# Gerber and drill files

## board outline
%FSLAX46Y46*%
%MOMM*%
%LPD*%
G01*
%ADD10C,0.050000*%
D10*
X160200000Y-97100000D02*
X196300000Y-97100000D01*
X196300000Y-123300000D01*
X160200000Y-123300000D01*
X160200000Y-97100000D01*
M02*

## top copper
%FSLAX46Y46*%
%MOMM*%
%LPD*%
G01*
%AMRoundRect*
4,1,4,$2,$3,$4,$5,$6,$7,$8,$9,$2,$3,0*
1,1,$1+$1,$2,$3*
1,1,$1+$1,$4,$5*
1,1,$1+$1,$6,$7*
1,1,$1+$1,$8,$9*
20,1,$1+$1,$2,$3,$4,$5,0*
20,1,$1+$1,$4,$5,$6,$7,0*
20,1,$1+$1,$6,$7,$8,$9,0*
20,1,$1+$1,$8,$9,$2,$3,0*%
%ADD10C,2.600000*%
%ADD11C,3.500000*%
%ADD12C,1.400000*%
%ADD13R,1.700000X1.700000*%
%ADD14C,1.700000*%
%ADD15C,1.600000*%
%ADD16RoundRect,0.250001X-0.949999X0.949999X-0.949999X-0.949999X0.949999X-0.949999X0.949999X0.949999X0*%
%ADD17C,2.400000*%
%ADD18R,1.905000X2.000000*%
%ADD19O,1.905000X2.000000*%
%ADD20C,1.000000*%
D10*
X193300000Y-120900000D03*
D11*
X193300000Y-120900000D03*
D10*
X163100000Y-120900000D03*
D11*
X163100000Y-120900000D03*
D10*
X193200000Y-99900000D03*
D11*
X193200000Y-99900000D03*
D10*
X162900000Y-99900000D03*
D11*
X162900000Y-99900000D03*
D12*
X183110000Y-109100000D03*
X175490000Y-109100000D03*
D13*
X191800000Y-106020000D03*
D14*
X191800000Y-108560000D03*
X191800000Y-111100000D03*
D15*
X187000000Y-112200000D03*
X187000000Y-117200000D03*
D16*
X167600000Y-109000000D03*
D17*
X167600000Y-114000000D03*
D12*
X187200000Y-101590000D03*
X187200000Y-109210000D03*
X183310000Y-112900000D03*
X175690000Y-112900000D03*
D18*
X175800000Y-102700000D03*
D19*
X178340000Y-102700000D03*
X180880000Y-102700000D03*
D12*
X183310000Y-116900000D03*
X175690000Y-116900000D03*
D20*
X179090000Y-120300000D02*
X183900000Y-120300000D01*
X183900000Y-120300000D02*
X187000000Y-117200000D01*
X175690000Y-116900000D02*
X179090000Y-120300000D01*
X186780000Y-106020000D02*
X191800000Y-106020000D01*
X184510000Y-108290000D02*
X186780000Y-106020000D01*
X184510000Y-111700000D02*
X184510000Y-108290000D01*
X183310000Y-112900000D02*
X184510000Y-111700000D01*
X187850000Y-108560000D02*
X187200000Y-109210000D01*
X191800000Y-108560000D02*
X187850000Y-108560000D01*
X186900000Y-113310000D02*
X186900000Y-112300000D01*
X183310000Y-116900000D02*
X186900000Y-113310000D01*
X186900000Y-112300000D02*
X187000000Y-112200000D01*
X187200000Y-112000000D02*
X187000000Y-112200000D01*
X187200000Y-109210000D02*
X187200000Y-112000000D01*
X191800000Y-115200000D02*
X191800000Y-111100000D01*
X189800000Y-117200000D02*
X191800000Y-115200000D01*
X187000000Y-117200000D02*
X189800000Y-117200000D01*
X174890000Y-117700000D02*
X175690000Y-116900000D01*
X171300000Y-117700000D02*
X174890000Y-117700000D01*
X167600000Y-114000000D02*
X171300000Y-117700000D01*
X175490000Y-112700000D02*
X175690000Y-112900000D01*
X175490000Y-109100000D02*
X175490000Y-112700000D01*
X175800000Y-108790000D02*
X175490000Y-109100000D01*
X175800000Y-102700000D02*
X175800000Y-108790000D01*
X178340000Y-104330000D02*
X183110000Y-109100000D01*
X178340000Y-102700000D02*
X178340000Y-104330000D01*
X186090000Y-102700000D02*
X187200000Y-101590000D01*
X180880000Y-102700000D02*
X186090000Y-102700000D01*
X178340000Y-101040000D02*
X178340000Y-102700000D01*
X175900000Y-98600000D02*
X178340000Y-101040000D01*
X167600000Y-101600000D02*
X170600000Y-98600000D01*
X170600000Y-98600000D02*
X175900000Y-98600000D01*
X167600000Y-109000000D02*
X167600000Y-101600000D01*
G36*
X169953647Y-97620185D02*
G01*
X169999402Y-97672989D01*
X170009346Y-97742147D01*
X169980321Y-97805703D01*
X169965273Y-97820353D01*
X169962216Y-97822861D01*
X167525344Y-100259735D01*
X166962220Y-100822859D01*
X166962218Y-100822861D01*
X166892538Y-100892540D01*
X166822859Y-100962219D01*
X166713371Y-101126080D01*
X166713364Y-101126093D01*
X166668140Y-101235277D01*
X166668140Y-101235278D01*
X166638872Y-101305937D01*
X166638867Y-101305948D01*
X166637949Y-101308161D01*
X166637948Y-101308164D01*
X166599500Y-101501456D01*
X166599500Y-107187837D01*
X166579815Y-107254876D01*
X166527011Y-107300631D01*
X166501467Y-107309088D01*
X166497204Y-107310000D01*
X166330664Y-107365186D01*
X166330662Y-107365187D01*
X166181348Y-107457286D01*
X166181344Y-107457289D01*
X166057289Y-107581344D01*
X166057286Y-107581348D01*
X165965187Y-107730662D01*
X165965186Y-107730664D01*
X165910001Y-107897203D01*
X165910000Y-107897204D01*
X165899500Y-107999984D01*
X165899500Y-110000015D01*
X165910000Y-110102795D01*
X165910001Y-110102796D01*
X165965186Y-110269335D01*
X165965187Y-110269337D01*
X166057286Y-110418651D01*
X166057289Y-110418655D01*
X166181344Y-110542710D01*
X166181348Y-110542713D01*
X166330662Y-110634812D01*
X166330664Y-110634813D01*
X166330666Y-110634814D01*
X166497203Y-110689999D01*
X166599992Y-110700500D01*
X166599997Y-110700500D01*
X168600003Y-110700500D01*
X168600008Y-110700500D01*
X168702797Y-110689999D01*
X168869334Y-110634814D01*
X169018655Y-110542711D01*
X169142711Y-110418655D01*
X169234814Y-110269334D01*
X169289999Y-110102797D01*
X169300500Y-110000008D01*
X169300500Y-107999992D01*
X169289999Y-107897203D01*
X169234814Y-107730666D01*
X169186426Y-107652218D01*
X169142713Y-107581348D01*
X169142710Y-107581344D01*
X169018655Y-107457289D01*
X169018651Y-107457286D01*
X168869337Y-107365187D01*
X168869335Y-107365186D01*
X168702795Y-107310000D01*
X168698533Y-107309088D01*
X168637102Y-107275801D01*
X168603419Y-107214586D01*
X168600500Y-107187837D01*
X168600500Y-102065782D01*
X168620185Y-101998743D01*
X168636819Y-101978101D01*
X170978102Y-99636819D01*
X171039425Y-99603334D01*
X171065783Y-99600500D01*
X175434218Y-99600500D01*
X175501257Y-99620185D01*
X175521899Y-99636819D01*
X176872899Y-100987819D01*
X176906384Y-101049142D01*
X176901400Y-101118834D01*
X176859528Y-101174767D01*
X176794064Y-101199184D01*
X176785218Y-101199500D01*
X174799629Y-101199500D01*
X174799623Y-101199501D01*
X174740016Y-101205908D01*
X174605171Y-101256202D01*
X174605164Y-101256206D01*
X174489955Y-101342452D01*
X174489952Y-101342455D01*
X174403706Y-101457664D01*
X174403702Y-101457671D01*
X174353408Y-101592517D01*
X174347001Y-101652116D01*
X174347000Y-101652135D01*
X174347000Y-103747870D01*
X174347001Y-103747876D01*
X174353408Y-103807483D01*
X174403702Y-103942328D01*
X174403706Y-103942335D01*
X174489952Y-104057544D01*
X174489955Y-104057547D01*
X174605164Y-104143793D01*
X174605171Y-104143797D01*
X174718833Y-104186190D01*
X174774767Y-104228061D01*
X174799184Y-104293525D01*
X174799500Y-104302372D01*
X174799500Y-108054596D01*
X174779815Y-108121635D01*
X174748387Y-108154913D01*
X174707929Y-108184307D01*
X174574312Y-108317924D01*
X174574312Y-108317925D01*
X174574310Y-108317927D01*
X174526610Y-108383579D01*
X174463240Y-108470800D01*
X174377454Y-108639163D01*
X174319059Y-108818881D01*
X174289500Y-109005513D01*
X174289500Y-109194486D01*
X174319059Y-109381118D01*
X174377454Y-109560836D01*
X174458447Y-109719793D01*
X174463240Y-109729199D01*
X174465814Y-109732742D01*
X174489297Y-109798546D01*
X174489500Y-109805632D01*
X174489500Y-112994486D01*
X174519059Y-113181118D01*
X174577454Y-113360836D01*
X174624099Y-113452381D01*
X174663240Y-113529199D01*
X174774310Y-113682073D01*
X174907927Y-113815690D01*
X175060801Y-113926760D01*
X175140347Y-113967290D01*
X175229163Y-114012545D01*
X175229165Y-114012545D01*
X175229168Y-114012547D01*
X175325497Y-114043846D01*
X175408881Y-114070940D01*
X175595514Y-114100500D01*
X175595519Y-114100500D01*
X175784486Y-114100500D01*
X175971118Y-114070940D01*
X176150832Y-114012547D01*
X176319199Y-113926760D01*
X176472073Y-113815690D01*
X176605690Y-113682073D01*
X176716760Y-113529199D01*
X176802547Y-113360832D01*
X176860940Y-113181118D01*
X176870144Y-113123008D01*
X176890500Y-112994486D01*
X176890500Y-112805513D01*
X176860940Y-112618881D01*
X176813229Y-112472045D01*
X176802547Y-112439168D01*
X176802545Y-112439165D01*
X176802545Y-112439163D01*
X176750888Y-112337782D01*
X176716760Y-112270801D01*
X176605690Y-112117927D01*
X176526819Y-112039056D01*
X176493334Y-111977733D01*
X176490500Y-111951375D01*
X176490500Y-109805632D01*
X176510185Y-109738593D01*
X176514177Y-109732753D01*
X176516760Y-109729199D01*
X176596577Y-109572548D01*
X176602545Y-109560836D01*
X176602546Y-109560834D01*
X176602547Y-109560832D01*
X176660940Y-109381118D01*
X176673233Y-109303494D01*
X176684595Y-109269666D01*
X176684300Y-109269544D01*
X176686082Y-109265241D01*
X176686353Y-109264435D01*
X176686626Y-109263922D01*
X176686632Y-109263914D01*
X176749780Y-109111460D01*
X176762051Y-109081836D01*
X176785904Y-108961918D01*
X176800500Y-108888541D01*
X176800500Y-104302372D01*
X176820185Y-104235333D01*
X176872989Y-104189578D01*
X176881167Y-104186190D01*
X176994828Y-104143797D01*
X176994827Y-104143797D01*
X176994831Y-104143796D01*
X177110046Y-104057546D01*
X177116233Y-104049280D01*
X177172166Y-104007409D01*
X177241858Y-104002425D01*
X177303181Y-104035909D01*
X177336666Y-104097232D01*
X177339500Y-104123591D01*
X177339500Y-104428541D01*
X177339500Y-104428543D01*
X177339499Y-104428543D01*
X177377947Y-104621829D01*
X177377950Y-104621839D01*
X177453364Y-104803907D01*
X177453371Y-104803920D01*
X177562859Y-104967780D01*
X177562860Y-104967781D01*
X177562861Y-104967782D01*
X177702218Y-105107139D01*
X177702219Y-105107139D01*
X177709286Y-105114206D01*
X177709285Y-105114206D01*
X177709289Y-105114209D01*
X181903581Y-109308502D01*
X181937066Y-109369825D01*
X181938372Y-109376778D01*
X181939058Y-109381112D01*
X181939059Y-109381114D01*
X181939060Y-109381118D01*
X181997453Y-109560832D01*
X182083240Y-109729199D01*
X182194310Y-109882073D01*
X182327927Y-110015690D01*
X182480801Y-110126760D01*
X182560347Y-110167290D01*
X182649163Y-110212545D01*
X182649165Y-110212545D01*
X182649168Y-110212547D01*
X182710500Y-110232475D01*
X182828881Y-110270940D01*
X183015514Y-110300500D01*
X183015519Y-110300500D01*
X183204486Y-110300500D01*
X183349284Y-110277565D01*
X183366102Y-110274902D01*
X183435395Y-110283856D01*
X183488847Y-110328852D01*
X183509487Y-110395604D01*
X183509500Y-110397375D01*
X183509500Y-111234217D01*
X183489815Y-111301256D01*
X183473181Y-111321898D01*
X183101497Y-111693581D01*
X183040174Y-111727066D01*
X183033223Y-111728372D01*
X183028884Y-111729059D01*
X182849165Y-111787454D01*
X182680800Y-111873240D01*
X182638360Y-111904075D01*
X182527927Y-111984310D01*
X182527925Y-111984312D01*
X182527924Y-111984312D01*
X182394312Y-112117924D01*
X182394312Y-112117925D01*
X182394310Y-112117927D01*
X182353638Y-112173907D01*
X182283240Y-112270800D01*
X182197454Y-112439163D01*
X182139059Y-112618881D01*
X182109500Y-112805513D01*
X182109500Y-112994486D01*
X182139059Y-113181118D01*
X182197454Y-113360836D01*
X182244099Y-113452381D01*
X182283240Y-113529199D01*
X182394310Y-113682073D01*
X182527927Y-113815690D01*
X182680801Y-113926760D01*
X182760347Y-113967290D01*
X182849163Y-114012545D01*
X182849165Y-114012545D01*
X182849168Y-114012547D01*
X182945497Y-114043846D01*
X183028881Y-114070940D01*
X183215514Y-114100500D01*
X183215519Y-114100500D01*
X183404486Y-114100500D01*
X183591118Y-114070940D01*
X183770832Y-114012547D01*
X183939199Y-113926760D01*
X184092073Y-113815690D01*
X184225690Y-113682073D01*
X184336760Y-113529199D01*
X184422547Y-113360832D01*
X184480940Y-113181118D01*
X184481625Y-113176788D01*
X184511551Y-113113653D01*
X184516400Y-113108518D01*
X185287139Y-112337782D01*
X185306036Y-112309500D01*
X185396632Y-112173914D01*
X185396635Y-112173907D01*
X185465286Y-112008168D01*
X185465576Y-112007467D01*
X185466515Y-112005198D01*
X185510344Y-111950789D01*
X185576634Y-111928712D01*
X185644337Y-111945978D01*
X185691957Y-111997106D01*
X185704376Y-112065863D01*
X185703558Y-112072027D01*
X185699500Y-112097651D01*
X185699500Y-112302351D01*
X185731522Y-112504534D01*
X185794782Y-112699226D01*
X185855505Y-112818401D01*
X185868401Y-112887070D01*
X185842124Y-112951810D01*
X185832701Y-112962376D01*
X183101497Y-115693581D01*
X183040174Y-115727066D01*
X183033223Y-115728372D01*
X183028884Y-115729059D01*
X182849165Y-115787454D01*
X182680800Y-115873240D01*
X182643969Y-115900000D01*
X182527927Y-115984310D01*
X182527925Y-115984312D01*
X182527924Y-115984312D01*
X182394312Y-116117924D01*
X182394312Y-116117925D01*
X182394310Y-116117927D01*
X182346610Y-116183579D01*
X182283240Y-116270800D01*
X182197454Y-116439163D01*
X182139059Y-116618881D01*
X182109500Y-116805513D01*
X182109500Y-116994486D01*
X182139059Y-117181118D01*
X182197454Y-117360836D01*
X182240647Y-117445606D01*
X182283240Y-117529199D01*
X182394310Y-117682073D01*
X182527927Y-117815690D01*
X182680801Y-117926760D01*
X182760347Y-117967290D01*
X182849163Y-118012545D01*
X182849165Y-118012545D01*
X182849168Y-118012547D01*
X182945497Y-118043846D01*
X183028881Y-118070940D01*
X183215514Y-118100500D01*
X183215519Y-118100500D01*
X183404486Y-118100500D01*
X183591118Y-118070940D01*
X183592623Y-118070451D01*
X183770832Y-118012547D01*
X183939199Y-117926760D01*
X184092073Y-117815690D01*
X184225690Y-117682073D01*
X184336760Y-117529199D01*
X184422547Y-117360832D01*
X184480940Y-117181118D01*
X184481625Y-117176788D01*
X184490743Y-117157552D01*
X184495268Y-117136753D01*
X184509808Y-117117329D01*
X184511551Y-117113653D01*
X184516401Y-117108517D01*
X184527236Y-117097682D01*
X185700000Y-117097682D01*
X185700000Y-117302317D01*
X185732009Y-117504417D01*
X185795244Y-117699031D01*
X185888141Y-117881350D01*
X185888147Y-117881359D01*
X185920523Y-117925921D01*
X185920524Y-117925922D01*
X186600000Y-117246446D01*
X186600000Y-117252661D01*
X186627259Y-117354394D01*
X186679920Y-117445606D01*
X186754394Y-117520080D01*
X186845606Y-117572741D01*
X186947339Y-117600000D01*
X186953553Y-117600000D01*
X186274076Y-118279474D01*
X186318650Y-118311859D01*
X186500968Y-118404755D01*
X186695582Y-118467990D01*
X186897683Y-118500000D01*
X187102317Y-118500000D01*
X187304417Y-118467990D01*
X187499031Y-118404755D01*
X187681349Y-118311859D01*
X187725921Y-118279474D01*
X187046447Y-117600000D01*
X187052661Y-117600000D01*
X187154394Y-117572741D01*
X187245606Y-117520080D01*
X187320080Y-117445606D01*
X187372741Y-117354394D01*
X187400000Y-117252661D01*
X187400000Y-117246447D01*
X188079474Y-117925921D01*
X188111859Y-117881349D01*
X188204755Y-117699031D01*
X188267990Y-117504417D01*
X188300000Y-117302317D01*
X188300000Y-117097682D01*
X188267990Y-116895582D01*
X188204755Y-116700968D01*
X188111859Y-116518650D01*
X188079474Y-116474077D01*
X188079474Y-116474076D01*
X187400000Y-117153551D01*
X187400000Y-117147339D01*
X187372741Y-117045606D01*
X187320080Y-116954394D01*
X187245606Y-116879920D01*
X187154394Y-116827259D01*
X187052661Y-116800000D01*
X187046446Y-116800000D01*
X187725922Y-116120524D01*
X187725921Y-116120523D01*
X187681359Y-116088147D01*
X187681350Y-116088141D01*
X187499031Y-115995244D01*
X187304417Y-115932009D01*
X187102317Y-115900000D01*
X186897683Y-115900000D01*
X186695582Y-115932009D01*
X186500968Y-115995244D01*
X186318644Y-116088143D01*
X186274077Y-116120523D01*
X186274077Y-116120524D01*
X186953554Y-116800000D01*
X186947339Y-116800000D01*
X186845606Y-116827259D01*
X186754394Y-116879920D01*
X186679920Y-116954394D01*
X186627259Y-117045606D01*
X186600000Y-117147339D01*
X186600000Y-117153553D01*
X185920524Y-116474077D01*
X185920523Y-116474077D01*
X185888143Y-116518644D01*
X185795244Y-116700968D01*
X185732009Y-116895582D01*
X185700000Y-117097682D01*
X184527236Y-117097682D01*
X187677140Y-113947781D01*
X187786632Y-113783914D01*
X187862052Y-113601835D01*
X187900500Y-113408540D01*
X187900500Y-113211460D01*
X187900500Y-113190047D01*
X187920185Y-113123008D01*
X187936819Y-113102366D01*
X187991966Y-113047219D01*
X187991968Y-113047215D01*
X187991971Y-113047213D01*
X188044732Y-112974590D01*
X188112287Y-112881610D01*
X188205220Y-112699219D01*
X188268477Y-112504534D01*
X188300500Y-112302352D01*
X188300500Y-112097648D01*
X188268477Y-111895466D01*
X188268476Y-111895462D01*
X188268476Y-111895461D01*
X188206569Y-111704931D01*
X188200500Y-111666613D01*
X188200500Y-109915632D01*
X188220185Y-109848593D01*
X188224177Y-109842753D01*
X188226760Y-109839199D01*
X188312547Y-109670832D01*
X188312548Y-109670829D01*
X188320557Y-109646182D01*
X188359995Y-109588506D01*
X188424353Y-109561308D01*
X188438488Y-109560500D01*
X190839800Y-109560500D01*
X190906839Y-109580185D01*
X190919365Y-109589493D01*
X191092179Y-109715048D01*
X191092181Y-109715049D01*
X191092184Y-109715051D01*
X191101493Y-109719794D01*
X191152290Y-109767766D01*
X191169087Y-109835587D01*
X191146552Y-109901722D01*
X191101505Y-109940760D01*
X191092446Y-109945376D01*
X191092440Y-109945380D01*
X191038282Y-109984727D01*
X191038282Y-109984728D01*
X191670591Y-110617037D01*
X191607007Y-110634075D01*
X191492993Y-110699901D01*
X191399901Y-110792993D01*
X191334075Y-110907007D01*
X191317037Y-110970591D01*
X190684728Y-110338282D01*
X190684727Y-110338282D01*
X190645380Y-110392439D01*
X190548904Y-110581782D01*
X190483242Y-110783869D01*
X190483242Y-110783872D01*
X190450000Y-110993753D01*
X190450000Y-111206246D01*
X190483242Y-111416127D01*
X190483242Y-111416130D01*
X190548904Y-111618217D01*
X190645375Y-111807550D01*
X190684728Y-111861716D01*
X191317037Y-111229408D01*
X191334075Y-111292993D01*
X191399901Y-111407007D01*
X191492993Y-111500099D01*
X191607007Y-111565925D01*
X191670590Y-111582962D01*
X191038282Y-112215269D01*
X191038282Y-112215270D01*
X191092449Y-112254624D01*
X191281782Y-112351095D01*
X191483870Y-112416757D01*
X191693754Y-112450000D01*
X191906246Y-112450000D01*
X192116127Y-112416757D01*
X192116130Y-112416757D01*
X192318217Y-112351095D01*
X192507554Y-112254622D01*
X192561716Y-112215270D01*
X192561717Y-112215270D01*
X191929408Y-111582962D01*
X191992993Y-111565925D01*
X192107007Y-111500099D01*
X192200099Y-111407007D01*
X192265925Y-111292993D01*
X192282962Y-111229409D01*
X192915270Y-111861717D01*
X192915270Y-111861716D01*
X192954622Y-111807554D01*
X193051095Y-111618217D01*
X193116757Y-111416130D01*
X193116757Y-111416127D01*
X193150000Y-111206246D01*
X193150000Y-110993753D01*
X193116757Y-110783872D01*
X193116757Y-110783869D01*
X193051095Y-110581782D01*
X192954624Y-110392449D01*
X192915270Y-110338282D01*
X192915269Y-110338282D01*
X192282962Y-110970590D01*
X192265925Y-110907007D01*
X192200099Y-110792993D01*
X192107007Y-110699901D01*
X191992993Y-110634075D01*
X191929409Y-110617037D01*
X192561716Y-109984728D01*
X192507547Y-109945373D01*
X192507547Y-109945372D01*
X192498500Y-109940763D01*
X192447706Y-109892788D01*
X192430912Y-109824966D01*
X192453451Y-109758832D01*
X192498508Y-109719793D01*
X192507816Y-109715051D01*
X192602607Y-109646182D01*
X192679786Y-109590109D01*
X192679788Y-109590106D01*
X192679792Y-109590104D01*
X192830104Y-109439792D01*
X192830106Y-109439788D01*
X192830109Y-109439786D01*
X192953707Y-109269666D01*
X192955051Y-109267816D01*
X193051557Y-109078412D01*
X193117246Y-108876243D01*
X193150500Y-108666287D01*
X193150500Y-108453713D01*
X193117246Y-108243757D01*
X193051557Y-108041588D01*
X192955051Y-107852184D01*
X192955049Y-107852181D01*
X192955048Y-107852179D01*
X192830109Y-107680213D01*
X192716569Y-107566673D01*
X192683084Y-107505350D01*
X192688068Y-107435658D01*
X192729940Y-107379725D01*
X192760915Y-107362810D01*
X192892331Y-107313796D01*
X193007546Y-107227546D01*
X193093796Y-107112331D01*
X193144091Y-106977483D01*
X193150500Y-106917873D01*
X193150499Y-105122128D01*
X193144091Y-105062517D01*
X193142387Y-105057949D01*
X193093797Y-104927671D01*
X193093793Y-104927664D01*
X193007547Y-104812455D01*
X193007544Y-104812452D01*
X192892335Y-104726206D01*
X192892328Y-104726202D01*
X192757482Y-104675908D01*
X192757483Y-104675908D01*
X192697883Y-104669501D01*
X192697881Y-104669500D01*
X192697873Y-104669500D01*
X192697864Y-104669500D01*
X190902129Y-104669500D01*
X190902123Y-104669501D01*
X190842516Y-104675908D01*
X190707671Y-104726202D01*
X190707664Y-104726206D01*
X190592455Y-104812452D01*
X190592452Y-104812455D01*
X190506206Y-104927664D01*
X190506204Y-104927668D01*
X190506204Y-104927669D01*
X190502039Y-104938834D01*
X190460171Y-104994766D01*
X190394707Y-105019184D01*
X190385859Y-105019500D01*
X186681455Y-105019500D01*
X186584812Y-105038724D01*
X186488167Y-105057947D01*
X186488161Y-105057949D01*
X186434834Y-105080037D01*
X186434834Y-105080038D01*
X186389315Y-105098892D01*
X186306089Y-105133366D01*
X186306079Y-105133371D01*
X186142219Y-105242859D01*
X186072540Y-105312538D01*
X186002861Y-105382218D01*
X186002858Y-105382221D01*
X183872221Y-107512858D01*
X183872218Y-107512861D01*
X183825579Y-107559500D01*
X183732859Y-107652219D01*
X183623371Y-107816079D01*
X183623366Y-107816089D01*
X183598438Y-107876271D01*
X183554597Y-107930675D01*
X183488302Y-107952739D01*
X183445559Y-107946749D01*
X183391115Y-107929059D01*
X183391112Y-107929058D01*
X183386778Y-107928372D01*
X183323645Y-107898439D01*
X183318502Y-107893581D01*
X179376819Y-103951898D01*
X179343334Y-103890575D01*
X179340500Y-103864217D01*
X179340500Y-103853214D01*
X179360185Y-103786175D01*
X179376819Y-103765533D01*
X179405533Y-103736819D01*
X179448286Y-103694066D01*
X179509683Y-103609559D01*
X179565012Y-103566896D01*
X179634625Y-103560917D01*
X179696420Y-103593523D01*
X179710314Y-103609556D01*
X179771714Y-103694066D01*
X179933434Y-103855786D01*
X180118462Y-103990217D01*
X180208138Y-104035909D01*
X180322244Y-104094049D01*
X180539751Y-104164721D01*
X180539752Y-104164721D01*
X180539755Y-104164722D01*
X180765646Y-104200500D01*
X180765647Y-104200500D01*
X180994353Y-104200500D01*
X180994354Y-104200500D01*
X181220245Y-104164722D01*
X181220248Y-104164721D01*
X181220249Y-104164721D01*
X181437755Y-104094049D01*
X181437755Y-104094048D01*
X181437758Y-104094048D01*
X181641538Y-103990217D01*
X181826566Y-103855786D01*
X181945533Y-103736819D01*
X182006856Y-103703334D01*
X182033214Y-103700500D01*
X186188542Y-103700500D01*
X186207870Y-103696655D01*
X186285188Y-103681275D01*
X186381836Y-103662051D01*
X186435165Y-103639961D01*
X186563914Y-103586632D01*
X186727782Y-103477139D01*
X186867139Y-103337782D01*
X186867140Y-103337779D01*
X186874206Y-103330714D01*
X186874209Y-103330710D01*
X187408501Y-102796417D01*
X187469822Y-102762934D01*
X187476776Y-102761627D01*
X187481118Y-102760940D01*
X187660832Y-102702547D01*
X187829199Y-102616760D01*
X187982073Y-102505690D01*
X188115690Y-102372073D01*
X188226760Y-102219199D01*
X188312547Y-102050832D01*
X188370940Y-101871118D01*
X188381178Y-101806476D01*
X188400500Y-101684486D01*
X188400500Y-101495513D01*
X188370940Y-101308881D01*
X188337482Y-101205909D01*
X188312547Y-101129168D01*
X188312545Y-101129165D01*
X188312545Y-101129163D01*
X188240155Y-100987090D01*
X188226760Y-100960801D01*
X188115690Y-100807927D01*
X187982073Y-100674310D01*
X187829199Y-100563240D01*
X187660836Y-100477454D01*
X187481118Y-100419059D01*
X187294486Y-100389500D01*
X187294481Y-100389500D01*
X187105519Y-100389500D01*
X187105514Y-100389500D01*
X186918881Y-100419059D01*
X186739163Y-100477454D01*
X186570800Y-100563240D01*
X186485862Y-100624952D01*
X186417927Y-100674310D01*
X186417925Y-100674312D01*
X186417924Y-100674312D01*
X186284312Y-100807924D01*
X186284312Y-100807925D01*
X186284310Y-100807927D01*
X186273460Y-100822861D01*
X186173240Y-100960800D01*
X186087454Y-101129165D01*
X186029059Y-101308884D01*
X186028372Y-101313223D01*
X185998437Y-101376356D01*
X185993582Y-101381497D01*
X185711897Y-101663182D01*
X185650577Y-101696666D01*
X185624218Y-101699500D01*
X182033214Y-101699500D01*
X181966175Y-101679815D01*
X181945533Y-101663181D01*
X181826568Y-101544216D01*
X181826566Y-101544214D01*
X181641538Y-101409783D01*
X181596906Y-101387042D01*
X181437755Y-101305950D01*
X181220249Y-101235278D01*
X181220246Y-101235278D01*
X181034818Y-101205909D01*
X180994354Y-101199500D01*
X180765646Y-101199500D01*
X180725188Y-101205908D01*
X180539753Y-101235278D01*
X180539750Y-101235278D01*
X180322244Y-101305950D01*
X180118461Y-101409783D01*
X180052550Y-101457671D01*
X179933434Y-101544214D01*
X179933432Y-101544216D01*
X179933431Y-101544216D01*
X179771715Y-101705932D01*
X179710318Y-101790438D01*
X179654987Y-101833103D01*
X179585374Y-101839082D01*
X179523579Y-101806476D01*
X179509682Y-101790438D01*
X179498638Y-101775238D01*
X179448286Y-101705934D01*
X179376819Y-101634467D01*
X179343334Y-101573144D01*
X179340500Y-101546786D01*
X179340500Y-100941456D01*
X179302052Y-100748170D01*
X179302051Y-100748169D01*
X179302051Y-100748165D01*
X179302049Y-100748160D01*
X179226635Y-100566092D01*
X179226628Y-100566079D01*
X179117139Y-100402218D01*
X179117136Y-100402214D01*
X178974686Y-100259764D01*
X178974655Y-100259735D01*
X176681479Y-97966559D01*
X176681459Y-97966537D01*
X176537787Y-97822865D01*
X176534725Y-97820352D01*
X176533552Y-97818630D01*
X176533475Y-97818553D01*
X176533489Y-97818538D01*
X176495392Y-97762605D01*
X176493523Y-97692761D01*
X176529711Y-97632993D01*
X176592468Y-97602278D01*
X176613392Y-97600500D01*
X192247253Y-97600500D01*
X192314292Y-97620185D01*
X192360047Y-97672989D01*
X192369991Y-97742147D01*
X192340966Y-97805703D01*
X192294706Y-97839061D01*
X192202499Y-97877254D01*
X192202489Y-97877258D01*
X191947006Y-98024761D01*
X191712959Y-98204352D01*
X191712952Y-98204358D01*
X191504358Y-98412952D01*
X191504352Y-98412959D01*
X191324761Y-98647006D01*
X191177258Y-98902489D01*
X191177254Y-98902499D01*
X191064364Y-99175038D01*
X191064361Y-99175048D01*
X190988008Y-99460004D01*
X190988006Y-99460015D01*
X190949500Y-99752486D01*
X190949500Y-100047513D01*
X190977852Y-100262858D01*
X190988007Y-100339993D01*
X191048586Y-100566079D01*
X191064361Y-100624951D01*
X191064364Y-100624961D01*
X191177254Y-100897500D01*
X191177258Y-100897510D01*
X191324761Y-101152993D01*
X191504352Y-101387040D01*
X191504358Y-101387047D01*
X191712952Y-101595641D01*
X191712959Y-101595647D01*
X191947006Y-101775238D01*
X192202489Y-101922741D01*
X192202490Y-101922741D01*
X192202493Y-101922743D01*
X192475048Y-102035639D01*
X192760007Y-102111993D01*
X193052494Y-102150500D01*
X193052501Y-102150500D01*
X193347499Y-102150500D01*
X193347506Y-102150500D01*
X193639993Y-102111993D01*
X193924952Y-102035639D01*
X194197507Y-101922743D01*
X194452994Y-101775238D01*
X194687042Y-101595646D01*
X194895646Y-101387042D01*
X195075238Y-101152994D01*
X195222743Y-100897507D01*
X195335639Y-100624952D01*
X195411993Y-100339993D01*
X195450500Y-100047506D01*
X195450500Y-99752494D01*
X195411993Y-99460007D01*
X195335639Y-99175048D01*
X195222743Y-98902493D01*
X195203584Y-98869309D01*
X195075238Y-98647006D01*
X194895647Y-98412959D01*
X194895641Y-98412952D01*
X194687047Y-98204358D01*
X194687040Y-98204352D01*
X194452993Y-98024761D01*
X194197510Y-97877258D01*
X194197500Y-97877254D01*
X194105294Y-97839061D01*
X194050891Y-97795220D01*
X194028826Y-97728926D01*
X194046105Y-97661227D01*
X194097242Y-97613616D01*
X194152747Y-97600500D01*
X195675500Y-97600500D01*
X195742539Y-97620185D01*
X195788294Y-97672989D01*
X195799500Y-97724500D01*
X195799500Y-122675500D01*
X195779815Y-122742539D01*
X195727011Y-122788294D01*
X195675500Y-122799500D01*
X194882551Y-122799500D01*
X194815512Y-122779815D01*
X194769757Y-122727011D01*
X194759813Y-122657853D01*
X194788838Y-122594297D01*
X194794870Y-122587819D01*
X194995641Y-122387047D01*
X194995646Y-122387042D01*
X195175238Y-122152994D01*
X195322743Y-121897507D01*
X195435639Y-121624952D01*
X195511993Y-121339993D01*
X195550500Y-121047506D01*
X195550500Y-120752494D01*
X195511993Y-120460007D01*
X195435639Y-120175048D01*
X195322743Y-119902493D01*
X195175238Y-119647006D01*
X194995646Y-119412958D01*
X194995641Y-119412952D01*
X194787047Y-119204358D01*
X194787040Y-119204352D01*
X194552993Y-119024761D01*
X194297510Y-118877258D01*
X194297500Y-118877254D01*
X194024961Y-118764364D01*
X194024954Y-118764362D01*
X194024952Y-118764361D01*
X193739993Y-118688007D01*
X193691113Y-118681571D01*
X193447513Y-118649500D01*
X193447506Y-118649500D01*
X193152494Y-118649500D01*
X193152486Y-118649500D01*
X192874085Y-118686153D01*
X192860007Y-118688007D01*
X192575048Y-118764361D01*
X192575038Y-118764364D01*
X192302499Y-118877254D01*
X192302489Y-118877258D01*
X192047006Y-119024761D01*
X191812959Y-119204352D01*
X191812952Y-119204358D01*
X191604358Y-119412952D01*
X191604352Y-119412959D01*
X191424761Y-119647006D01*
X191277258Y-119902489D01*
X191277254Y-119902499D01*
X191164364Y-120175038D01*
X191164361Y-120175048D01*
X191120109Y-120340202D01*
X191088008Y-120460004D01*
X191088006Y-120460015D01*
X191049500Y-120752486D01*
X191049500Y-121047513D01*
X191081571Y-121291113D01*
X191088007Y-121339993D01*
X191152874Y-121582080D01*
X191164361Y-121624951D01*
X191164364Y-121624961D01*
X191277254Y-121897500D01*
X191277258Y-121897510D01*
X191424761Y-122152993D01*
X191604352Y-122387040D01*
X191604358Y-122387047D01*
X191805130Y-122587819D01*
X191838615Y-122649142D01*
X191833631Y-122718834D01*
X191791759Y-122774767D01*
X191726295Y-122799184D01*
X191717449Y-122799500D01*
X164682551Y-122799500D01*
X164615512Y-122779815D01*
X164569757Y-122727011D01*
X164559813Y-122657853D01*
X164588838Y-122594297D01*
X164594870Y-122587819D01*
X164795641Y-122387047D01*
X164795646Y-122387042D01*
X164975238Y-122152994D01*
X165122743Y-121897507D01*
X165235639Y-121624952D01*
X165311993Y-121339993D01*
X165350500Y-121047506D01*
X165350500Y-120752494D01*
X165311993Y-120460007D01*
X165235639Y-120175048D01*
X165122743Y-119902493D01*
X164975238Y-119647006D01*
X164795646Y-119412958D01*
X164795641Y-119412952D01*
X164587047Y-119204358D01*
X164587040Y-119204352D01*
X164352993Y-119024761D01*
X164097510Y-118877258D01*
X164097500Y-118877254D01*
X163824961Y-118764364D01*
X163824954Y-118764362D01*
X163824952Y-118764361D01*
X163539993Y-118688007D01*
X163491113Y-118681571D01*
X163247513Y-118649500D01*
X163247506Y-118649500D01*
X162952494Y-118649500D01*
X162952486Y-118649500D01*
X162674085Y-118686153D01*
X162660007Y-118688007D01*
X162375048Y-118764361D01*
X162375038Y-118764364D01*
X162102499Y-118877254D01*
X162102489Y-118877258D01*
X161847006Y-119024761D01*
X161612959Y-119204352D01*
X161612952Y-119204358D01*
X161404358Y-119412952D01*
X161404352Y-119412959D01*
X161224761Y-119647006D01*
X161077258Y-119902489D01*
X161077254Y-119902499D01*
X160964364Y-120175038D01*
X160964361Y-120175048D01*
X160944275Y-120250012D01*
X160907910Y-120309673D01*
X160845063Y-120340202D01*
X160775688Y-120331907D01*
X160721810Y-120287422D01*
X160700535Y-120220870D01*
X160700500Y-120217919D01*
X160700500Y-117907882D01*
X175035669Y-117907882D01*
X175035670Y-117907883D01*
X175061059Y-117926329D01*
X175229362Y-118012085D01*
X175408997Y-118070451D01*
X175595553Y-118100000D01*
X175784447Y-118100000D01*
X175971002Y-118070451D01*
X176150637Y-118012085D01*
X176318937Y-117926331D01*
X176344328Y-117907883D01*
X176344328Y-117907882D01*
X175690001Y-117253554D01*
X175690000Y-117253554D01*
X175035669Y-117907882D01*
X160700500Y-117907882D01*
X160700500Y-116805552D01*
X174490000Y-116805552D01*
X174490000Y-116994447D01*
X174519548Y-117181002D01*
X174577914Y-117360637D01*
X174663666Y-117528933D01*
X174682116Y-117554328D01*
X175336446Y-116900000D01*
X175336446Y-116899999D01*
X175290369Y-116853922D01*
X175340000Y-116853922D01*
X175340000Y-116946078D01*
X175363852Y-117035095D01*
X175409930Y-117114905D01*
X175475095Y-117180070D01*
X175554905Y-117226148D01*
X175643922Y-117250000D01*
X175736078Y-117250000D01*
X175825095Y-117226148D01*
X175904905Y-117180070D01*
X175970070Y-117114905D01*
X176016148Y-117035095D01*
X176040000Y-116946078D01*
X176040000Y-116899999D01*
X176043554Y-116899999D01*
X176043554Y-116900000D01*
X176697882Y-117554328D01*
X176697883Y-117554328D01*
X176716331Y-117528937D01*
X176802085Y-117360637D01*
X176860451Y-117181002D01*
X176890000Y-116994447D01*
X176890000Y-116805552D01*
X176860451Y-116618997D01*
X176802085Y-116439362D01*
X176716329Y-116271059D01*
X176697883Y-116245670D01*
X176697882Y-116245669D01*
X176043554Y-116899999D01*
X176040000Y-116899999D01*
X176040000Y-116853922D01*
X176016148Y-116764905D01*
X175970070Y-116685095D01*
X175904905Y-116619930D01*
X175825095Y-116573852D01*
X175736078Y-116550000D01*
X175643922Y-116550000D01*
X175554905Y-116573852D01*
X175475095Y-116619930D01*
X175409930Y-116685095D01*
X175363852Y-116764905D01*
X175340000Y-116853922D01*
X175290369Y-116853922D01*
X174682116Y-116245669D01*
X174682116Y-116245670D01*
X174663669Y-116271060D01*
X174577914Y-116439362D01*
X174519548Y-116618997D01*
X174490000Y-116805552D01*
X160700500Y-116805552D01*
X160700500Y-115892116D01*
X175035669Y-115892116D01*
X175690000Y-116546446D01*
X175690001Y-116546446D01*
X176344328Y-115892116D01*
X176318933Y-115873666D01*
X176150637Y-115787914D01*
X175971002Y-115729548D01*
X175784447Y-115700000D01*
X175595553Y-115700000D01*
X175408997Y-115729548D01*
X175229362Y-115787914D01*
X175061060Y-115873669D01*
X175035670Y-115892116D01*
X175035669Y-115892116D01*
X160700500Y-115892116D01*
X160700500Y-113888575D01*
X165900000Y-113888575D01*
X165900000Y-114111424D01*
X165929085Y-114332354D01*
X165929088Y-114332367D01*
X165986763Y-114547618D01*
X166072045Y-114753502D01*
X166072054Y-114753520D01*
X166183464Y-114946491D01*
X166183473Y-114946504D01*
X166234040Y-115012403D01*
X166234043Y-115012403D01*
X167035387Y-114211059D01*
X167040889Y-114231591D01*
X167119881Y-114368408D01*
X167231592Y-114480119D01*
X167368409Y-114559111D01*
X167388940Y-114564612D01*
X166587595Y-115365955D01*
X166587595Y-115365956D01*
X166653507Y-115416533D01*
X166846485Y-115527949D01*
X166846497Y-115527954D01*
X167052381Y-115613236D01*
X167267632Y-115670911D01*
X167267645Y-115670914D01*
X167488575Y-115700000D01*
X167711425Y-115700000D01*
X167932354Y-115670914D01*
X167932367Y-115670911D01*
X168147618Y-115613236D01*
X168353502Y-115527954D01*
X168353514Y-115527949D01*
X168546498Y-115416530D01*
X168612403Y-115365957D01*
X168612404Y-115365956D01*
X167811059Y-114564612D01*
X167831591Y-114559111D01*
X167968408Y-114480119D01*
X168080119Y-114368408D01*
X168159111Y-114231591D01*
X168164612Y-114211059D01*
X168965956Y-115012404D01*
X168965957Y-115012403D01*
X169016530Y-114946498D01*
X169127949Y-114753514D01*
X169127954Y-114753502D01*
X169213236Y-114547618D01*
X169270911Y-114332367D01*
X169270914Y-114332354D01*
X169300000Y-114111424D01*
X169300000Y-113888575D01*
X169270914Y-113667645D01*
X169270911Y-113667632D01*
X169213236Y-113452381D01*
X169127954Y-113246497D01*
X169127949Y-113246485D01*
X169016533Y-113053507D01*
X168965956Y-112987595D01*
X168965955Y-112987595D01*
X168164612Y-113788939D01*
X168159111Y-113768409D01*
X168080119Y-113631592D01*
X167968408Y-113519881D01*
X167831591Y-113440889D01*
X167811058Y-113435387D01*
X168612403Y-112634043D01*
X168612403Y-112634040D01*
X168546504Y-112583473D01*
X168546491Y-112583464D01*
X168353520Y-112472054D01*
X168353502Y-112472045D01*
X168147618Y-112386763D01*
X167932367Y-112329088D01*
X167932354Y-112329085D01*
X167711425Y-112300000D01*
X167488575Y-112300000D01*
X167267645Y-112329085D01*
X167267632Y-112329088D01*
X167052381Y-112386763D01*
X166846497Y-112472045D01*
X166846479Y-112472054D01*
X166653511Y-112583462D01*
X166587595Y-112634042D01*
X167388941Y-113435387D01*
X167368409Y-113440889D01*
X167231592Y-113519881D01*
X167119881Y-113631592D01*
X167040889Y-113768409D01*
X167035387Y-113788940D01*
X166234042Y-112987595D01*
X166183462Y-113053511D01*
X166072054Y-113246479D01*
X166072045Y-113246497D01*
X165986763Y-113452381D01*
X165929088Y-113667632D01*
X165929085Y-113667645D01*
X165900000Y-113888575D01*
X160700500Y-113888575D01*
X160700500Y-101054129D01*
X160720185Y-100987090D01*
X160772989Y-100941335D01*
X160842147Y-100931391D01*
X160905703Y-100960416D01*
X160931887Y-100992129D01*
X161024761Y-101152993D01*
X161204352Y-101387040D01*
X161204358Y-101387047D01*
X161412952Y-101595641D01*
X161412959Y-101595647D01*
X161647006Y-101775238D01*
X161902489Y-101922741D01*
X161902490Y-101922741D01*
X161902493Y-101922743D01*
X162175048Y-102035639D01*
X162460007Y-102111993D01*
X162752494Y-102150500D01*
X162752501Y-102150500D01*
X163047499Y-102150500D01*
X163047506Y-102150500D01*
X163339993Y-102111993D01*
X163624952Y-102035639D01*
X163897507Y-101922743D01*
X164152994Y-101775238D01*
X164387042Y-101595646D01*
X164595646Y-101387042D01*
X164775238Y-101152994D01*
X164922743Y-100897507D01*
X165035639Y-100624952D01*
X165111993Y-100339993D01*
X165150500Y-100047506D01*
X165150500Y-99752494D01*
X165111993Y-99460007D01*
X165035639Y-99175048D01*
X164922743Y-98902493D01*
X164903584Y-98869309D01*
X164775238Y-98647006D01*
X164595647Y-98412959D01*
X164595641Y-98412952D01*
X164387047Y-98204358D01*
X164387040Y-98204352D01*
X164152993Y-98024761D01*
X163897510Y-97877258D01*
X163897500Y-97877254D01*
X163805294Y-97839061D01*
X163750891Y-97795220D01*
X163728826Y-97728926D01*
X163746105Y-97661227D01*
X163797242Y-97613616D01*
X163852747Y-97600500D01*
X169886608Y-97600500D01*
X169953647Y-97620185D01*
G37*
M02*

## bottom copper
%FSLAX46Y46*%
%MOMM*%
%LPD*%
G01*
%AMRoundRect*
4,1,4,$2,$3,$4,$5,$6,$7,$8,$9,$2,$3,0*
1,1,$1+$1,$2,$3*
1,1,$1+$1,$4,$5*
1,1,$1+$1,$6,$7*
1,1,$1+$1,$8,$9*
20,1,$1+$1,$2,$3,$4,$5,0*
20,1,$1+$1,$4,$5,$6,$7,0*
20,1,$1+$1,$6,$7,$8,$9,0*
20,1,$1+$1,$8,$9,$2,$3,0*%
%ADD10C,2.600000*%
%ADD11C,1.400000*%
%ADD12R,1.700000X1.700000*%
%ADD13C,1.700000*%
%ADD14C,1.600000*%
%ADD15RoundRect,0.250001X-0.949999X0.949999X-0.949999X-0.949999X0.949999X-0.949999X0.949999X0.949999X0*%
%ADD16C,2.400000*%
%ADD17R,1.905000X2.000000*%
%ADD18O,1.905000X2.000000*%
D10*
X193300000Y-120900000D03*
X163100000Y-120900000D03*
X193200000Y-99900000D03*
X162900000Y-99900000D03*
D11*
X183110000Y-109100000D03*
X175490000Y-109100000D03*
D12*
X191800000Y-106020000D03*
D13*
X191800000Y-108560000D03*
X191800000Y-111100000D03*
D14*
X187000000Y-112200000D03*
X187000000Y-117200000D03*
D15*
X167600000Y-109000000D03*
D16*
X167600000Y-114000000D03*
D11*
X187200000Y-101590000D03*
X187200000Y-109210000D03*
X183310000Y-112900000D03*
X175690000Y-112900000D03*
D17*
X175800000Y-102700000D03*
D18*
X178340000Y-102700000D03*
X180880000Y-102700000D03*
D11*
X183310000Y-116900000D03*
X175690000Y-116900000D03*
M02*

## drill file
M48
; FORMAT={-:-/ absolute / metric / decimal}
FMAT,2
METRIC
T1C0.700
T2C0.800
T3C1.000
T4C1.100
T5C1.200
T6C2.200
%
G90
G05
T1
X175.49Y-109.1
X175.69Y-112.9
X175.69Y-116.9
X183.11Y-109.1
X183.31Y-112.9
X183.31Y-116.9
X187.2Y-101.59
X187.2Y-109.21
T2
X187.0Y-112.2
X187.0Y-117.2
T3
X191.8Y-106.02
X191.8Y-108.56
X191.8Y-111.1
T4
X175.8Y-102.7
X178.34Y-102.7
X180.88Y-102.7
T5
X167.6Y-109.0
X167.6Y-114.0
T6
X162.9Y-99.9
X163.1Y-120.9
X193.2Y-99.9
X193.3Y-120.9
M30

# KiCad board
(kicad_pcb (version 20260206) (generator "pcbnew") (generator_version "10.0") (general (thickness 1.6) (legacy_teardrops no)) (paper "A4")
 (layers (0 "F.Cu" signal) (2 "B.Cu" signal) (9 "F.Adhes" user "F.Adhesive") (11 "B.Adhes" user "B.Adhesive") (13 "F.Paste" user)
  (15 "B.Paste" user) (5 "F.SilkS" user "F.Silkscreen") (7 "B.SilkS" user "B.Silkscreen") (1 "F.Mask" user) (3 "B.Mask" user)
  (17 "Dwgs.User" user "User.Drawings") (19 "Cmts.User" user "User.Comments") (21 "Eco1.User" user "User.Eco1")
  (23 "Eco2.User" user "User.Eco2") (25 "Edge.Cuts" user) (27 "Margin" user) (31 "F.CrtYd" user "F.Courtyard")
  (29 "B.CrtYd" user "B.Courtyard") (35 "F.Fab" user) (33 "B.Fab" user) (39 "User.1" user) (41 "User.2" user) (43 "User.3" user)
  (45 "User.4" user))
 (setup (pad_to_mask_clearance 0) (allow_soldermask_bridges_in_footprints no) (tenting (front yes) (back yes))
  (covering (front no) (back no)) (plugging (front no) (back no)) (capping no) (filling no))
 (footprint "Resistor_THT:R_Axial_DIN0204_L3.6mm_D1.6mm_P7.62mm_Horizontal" (layer "F.Cu") (at 183.11 109.1 180)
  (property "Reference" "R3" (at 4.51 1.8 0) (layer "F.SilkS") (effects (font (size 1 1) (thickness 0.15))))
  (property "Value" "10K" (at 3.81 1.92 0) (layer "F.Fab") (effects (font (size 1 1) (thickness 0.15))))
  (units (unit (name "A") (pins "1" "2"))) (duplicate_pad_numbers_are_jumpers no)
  (pad "1" thru_hole circle (at 0 0 180) (size 1.4 1.4) (drill 0.7) (layers "*.Cu" "*.Mask") (remove_unused_layers no)
   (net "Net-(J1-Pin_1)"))
  (pad "2" thru_hole circle (at 7.62 0 180) (size 1.4 1.4) (drill 0.7) (layers "*.Cu" "*.Mask") (remove_unused_layers no) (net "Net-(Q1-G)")))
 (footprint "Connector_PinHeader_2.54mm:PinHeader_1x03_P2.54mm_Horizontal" (layer "F.Cu") (at 191.8 106.02)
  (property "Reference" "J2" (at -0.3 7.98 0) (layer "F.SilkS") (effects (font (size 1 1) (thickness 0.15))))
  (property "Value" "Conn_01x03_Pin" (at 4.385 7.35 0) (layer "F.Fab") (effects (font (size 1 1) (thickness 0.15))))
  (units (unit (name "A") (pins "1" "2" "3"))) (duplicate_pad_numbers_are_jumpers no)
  (pad "1" thru_hole rect (at 0 0) (size 1.7 1.7) (drill 1) (layers "*.Cu" "*.Mask") (remove_unused_layers no) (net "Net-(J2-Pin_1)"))
  (pad "2" thru_hole circle (at 0 2.54) (size 1.7 1.7) (drill 1) (layers "*.Cu" "*.Mask") (remove_unused_layers no) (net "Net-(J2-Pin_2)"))
  (pad "3" thru_hole circle (at 0 5.08) (size 1.7 1.7) (drill 1) (layers "*.Cu" "*.Mask") (remove_unused_layers no) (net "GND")))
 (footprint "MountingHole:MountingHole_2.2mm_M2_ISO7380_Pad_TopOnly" (layer "F.Cu") (at 162.9 99.9)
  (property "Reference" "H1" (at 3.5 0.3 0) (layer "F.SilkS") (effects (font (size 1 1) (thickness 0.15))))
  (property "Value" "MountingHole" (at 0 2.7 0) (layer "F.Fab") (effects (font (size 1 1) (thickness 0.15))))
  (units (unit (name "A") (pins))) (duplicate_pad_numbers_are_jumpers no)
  (pad "1" thru_hole circle (at 0 0) (size 2.6 2.6) (drill 2.2) (layers "*.Cu" "*.Mask") (remove_unused_layers no) (zone_connect 2))
  (pad "1" connect circle (at 0 0) (size 3.5 3.5) (layers "F.Cu" "F.Mask") (zone_connect 2)))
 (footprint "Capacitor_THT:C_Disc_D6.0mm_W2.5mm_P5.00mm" (layer "F.Cu") (at 187 112.2 -90)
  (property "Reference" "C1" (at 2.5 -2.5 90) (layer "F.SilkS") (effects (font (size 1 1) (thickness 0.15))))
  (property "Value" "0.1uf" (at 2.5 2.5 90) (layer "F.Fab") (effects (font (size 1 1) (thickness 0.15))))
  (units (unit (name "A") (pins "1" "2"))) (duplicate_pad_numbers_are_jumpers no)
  (pad "1" thru_hole circle (at 0 0 270) (size 1.6 1.6) (drill 0.8) (layers "*.Cu" "*.Mask") (remove_unused_layers no)
   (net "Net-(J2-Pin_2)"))
  (pad "2" thru_hole circle (at 5 0 270) (size 1.6 1.6) (drill 0.8) (layers "*.Cu" "*.Mask") (remove_unused_layers no) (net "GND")))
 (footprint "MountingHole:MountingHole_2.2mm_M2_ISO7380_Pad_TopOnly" (layer "F.Cu") (at 193.3 120.9)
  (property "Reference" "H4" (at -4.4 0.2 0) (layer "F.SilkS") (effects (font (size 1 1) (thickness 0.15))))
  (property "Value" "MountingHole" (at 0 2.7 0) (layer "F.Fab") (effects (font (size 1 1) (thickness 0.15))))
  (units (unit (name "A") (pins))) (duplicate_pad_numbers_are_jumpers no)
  (pad "1" thru_hole circle (at 0 0) (size 2.6 2.6) (drill 2.2) (layers "*.Cu" "*.Mask") (remove_unused_layers no) (zone_connect 2))
  (pad "1" connect circle (at 0 0) (size 3.5 3.5) (layers "F.Cu" "F.Mask") (zone_connect 2)))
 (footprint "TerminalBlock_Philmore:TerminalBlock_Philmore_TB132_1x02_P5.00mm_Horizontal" (layer "F.Cu") (at 167.6 109 -90)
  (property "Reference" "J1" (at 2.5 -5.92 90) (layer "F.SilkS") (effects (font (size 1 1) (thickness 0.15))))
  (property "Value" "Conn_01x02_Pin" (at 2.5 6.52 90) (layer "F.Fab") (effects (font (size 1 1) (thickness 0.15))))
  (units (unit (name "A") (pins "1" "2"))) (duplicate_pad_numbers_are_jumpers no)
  (pad "1" thru_hole roundrect (at 0 0 270) (size 2.4 2.4) (drill 1.2) (layers "*.Cu" "*.Mask") (remove_unused_layers no)
   (roundrect_rratio 0.104167) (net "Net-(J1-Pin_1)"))
  (pad "2" thru_hole circle (at 5 0 270) (size 2.4 2.4) (drill 1.2) (layers "*.Cu" "*.Mask") (remove_unused_layers no) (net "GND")))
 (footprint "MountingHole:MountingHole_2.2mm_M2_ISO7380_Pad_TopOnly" (layer "F.Cu") (at 193.2 99.9)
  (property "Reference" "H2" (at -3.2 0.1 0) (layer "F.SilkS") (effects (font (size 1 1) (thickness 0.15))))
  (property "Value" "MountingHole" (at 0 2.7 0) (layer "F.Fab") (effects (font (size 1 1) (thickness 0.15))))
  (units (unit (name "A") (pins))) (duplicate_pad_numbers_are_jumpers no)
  (pad "1" thru_hole circle (at 0 0) (size 2.6 2.6) (drill 2.2) (layers "*.Cu" "*.Mask") (remove_unused_layers no) (zone_connect 2))
  (pad "1" connect circle (at 0 0) (size 3.5 3.5) (layers "F.Cu" "F.Mask") (zone_connect 2)))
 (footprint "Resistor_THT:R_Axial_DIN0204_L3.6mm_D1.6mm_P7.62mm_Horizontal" (layer "F.Cu") (at 187.2 101.59 -90)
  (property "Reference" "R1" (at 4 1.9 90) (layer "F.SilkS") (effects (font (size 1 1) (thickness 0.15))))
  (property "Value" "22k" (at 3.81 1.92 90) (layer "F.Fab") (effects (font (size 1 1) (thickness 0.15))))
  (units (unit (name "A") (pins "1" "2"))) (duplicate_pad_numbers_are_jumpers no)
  (pad "1" thru_hole circle (at 0 0 270) (size 1.4 1.4) (drill 0.7) (layers "*.Cu" "*.Mask") (remove_unused_layers no) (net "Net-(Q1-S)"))
  (pad "2" thru_hole circle (at 7.62 0 270) (size 1.4 1.4) (drill 0.7) (layers "*.Cu" "*.Mask") (remove_unused_layers no)
   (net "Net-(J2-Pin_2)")))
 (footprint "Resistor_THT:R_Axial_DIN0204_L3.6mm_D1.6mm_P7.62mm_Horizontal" (layer "F.Cu") (at 183.31 112.9 180)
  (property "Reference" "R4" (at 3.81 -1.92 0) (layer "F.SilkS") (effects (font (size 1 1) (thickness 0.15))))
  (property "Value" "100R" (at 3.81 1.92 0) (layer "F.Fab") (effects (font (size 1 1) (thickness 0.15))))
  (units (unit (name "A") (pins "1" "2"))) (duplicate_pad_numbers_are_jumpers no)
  (pad "1" thru_hole circle (at 0 0 180) (size 1.4 1.4) (drill 0.7) (layers "*.Cu" "*.Mask") (remove_unused_layers no)
   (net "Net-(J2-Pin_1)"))
  (pad "2" thru_hole circle (at 7.62 0 180) (size 1.4 1.4) (drill 0.7) (layers "*.Cu" "*.Mask") (remove_unused_layers no) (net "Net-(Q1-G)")))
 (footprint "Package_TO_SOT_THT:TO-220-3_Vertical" (layer "F.Cu") (at 175.8 102.7)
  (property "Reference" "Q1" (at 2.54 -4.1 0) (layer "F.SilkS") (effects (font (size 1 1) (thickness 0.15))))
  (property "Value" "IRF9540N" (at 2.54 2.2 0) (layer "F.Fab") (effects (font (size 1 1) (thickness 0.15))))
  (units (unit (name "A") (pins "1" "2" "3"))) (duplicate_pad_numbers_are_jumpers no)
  (pad "1" thru_hole rect (at 0 0) (size 1.905 2) (drill 1.1) (layers "*.Cu" "*.Mask") (remove_unused_layers no) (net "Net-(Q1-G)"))
  (pad "2" thru_hole oval (at 2.54 0) (size 1.905 2) (drill 1.1) (layers "*.Cu" "*.Mask") (remove_unused_layers no) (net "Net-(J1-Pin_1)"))
  (pad "3" thru_hole oval (at 5.08 0) (size 1.905 2) (drill 1.1) (layers "*.Cu" "*.Mask") (remove_unused_layers no) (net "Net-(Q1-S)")))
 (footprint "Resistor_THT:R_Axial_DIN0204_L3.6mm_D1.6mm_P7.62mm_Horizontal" (layer "F.Cu") (at 183.31 116.9 180)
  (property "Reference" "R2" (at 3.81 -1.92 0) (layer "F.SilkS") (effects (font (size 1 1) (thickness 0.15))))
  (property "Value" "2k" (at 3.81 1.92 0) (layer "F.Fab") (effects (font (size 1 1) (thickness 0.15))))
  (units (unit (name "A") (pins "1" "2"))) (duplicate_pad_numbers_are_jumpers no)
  (pad "1" thru_hole circle (at 0 0 180) (size 1.4 1.4) (drill 0.7) (layers "*.Cu" "*.Mask") (remove_unused_layers no)
   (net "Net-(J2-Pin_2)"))
  (pad "2" thru_hole circle (at 7.62 0 180) (size 1.4 1.4) (drill 0.7) (layers "*.Cu" "*.Mask") (remove_unused_layers no) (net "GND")))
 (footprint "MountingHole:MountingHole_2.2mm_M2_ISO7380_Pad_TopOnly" (layer "F.Cu") (at 163.1 120.9)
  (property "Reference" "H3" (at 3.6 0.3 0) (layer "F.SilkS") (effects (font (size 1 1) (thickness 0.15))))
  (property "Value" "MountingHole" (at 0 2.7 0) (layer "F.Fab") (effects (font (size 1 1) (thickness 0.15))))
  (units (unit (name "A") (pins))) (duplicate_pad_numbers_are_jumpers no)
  (pad "1" thru_hole circle (at 0 0) (size 2.6 2.6) (drill 2.2) (layers "*.Cu" "*.Mask") (remove_unused_layers no) (zone_connect 2))
  (pad "1" connect circle (at 0 0) (size 3.5 3.5) (layers "F.Cu" "F.Mask") (zone_connect 2)))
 (gr_rect (start 160.2 97.1) (end 196.3 123.3) (stroke (width 0.05) (type default)) (fill no) (layer "Edge.Cuts"))
 (segment (start 167.6 101.6) (end 170.6 98.6) (width 1) (layer "F.Cu") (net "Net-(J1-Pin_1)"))
 (segment (start 178.34 101.04) (end 178.34 102.7) (width 1) (layer "F.Cu") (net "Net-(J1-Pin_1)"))
 (segment (start 178.34 104.33) (end 183.11 109.1) (width 1) (layer "F.Cu") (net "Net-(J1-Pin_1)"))
 (segment (start 175.9 98.6) (end 178.34 101.04) (width 1) (layer "F.Cu") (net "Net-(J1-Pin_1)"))
 (segment (start 178.34 102.7) (end 178.34 104.33) (width 1) (layer "F.Cu") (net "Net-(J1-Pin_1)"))
 (segment (start 170.6 98.6) (end 175.9 98.6) (width 1) (layer "F.Cu") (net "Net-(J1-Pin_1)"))
 (segment (start 167.6 109) (end 167.6 101.6) (width 1) (layer "F.Cu") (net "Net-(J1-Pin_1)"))
 (segment (start 175.8 108.79) (end 175.49 109.1) (width 1) (layer "F.Cu") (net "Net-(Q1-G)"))
 (segment (start 175.8 102.7) (end 175.8 108.79) (width 1) (layer "F.Cu") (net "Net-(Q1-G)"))
 (segment (start 175.49 109.1) (end 175.49 112.7) (width 1) (layer "F.Cu") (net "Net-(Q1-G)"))
 (segment (start 175.49 112.7) (end 175.69 112.9) (width 1) (layer "F.Cu") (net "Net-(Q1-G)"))
 (segment (start 184.51 108.29) (end 186.78 106.02) (width 1) (layer "F.Cu") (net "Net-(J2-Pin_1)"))
 (segment (start 184.51 111.7) (end 184.51 108.29) (width 1) (layer "F.Cu") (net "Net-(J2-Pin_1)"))
 (segment (start 186.78 106.02) (end 191.8 106.02) (width 1) (layer "F.Cu") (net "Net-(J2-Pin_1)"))
 (segment (start 183.31 112.9) (end 184.51 111.7) (width 1) (layer "F.Cu") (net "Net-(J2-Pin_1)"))
 (segment (start 191.8 108.56) (end 187.85 108.56) (width 1) (layer "F.Cu") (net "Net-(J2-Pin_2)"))
 (segment (start 186.9 113.31) (end 186.9 112.3) (width 1) (layer "F.Cu") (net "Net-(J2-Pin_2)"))
 (segment (start 183.31 116.9) (end 186.9 113.31) (width 1) (layer "F.Cu") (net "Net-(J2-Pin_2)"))
 (segment (start 187.85 108.56) (end 187.2 109.21) (width 1) (layer "F.Cu") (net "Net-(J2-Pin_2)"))
 (segment (start 186.9 112.3) (end 187 112.2) (width 1) (layer "F.Cu") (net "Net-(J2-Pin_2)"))
 (segment (start 187.2 112) (end 187 112.2) (width 1) (layer "F.Cu") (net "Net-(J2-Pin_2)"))
 (segment (start 187.2 109.21) (end 187.2 112) (width 1) (layer "F.Cu") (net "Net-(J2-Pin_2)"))
 (segment (start 179.09 120.3) (end 183.9 120.3) (width 1) (layer "F.Cu") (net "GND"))
 (segment (start 167.6 114) (end 171.3 117.7) (width 1) (layer "F.Cu") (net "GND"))
 (segment (start 189.8 117.2) (end 191.8 115.2) (width 1) (layer "F.Cu") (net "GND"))
 (segment (start 174.89 117.7) (end 175.69 116.9) (width 1) (layer "F.Cu") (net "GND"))
 (segment (start 187 117.2) (end 189.8 117.2) (width 1) (layer "F.Cu") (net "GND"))
 (segment (start 191.8 115.2) (end 191.8 111.1) (width 1) (layer "F.Cu") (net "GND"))
 (segment (start 183.9 120.3) (end 187 117.2) (width 1) (layer "F.Cu") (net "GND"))
 (segment (start 171.3 117.7) (end 174.89 117.7) (width 1) (layer "F.Cu") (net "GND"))
 (segment (start 175.69 116.9) (end 179.09 120.3) (width 1) (layer "F.Cu") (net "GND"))
 (segment (start 180.88 102.7) (end 186.09 102.7) (width 1) (layer "F.Cu") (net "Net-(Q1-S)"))
 (segment (start 186.09 102.7) (end 187.2 101.59) (width 1) (layer "F.Cu") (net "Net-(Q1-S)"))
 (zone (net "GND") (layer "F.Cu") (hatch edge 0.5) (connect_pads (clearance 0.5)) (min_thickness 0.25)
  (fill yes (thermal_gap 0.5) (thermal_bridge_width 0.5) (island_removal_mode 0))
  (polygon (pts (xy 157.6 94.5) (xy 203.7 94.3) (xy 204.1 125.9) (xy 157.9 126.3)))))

